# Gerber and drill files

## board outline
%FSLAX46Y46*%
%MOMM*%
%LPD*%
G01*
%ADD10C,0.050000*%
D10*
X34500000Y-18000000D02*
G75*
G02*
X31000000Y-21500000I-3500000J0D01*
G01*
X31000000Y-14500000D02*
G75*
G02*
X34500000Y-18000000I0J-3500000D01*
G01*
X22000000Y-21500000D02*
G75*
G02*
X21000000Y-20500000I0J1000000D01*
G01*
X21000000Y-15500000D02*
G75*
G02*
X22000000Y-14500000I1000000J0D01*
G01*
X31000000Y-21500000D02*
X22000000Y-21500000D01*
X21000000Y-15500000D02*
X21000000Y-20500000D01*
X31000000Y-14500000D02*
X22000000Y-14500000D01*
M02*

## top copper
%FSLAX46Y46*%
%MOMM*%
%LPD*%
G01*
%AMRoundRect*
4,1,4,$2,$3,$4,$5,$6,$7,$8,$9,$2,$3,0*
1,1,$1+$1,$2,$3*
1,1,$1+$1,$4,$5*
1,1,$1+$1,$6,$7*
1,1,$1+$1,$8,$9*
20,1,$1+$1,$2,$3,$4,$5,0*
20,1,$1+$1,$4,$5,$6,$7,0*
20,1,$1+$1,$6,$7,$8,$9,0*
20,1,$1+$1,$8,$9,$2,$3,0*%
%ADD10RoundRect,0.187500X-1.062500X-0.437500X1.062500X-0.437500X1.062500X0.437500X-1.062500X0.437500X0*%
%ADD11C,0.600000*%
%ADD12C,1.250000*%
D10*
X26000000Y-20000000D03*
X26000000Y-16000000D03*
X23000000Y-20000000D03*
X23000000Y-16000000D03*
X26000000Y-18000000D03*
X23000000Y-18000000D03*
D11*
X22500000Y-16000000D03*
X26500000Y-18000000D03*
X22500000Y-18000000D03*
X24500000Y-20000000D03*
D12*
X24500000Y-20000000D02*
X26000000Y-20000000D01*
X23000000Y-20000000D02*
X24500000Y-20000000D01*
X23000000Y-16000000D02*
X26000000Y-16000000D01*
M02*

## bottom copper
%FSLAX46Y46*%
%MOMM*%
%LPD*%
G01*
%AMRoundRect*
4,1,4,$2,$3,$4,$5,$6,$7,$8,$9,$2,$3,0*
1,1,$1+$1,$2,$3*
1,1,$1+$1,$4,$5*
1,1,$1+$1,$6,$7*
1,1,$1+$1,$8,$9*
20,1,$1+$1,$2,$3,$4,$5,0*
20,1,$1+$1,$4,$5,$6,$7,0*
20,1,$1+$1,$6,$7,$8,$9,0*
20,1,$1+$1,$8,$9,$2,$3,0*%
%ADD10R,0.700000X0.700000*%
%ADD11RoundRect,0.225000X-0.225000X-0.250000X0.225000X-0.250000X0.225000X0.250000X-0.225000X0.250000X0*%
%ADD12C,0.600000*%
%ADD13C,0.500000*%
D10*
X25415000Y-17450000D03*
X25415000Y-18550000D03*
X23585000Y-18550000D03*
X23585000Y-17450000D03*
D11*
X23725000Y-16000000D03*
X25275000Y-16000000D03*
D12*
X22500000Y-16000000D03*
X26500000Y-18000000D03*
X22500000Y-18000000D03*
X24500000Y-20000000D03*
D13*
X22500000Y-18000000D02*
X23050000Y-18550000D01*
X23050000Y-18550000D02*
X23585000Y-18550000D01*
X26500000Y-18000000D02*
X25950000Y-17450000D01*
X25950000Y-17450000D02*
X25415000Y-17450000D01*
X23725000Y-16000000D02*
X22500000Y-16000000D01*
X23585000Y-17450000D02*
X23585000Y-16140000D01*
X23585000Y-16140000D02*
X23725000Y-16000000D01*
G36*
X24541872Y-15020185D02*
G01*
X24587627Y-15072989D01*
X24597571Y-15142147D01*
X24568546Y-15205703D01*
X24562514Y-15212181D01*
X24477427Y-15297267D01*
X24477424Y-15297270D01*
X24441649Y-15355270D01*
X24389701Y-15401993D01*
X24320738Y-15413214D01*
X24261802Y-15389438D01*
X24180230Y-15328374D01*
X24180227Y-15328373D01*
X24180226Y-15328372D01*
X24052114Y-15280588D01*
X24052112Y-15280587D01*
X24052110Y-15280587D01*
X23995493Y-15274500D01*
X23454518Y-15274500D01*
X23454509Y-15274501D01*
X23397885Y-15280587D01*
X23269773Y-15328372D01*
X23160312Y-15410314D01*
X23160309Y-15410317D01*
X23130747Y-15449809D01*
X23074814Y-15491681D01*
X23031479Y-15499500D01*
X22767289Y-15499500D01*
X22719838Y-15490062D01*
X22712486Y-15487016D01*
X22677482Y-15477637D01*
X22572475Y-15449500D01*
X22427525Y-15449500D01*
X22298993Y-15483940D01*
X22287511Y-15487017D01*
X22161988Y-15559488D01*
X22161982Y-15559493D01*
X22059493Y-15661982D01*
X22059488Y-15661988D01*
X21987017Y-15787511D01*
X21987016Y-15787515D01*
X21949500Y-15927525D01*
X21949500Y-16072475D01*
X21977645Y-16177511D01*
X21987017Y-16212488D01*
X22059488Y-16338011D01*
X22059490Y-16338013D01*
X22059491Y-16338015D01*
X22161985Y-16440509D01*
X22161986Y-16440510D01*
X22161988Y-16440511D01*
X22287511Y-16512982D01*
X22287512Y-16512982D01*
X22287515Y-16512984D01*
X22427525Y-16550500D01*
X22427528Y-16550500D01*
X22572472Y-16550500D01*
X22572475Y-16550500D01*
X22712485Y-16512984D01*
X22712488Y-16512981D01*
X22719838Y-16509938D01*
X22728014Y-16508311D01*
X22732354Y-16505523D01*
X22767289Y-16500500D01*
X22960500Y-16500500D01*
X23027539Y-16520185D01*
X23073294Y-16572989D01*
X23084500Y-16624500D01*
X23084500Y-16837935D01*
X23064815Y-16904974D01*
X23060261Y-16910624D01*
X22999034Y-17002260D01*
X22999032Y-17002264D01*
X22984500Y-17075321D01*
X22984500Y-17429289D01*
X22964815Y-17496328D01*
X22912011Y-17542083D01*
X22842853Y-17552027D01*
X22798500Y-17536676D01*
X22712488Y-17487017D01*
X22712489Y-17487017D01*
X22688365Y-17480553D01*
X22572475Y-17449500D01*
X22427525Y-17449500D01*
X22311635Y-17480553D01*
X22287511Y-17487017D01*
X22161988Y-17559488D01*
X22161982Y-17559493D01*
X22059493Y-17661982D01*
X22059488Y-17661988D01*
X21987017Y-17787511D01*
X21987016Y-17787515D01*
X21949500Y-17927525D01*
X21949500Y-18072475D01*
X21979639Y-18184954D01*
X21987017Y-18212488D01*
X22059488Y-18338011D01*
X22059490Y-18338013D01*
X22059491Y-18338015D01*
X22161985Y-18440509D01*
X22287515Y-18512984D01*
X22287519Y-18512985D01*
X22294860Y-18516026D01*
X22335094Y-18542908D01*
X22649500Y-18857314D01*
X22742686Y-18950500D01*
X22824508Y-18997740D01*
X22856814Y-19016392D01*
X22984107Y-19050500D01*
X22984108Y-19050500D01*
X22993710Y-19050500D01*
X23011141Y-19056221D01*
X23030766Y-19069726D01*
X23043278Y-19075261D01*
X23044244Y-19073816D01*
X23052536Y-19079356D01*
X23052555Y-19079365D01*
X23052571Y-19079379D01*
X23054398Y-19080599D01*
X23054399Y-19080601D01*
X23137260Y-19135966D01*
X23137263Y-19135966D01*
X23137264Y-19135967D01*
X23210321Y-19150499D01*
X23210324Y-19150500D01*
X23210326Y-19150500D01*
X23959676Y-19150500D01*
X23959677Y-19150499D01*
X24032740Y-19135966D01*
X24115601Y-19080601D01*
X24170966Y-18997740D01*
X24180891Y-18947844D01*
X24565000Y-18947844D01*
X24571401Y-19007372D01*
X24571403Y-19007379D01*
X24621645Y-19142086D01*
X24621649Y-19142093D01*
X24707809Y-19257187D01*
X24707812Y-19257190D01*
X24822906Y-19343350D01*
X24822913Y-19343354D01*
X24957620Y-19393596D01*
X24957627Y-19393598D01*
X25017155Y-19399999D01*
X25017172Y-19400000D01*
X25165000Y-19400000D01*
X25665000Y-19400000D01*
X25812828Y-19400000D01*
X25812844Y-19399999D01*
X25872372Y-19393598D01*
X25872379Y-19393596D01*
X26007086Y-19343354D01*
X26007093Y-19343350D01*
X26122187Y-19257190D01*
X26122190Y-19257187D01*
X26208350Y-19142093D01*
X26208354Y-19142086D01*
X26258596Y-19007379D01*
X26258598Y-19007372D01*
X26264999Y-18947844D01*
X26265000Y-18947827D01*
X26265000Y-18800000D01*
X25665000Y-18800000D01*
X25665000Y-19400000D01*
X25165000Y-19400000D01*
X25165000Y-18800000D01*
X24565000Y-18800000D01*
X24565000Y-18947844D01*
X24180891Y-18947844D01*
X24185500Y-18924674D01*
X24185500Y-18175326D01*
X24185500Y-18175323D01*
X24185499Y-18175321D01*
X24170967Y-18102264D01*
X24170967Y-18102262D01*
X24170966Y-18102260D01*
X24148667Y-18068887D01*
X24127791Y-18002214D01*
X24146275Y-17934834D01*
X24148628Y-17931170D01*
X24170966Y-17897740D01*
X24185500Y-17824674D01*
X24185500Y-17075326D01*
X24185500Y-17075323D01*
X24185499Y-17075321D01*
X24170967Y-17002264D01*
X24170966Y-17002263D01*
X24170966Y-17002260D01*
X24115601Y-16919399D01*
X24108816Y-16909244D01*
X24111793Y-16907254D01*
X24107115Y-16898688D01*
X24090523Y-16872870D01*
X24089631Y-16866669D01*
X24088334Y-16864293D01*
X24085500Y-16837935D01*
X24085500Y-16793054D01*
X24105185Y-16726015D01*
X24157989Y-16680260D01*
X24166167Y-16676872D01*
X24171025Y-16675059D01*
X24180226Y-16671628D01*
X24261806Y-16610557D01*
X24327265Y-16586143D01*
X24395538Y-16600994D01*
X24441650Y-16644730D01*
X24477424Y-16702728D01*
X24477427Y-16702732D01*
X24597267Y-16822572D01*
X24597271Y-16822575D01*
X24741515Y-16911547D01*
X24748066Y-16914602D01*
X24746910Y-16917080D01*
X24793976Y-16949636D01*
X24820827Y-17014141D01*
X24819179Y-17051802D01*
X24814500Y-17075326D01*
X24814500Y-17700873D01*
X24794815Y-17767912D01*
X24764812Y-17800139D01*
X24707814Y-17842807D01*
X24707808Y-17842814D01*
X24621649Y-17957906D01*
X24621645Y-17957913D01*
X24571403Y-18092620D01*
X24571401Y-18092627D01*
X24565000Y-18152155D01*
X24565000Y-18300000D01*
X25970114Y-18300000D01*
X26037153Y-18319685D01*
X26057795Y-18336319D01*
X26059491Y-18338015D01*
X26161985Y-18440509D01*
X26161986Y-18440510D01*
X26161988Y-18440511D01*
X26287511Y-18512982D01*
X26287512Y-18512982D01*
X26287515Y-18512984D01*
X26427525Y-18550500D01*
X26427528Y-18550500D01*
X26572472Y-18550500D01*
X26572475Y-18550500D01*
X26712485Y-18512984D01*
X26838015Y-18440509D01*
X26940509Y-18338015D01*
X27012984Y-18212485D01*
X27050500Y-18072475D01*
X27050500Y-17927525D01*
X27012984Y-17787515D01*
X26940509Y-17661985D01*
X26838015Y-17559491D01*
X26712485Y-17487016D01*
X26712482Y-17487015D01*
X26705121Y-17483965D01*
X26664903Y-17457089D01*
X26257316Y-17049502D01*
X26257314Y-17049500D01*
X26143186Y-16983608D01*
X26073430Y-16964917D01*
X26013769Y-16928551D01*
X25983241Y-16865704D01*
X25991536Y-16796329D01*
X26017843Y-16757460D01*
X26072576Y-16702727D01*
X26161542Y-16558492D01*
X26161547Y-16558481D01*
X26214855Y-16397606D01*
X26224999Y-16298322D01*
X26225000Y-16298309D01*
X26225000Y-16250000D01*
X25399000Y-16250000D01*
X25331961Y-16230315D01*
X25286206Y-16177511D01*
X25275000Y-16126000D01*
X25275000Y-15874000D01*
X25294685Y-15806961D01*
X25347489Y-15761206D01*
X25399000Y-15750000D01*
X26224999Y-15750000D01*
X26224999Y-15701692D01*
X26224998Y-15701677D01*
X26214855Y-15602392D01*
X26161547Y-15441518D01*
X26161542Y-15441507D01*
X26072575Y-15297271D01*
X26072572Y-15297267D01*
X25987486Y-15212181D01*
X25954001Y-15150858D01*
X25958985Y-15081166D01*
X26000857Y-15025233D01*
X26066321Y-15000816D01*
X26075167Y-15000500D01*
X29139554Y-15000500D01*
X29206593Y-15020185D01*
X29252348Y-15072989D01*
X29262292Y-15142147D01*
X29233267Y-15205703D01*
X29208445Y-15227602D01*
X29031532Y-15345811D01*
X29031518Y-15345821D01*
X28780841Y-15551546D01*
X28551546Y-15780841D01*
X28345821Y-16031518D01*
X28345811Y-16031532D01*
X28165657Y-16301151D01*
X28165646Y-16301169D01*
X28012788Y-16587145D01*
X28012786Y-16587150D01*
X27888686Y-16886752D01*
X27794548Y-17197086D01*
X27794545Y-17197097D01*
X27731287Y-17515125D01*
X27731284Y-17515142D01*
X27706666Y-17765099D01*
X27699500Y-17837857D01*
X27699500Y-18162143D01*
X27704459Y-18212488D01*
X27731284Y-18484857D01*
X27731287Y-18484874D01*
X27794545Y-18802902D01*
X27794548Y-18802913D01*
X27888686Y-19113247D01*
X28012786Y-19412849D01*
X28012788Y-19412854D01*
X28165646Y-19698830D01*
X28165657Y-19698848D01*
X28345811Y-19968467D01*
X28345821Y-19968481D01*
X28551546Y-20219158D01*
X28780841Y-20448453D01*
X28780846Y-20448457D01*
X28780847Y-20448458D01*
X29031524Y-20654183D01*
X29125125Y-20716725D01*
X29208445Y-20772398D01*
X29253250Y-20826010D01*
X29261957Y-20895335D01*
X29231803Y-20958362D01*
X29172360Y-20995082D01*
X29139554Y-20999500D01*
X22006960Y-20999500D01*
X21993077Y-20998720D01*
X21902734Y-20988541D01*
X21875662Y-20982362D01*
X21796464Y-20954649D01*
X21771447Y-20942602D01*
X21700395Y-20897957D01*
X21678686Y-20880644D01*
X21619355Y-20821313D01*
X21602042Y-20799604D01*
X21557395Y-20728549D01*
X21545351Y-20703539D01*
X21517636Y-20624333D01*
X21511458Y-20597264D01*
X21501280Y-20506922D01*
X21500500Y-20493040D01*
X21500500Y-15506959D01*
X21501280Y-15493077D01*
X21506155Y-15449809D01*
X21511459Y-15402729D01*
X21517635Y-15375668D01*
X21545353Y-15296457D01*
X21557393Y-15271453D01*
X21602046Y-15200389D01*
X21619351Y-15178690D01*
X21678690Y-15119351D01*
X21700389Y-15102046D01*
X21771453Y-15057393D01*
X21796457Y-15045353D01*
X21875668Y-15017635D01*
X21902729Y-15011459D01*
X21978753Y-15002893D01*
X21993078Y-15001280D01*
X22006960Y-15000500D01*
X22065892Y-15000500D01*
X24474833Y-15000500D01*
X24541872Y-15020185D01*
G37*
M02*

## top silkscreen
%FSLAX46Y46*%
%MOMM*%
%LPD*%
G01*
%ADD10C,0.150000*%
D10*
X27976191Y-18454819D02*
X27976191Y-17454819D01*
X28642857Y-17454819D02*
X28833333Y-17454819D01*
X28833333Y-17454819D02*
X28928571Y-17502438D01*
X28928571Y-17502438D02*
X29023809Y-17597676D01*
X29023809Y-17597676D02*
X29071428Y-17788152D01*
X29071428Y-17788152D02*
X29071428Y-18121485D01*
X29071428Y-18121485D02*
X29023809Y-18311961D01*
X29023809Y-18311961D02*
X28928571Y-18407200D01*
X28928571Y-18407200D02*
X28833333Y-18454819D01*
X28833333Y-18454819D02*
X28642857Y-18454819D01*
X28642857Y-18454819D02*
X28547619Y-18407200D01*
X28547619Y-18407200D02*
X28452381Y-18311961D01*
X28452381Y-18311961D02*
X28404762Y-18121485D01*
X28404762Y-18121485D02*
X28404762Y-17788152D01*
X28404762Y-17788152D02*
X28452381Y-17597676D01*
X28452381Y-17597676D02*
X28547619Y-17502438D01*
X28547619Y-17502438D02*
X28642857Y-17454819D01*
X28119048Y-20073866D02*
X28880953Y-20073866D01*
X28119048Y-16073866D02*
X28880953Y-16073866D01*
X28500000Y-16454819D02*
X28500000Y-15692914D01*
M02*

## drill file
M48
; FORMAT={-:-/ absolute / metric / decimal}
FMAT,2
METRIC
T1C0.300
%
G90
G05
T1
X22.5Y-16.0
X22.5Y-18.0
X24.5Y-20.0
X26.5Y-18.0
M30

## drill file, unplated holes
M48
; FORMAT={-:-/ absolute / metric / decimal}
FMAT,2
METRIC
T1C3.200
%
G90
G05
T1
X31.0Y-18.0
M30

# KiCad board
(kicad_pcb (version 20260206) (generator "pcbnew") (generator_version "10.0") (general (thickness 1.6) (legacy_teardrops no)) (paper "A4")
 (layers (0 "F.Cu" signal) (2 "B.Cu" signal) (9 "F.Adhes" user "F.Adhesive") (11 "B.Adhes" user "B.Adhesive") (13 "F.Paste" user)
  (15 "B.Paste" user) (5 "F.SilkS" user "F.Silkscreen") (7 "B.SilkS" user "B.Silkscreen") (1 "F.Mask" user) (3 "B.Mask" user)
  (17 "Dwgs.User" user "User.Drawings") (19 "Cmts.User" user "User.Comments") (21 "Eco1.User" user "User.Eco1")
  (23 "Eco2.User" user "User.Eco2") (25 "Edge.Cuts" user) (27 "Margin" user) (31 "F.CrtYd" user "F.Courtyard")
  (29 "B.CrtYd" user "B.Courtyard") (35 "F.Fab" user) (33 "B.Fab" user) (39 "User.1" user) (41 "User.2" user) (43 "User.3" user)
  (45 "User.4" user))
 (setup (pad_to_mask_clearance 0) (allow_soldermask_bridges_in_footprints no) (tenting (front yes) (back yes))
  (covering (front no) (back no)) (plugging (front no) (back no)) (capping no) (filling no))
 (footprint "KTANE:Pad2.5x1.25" (layer "F.Cu") (at 26 16)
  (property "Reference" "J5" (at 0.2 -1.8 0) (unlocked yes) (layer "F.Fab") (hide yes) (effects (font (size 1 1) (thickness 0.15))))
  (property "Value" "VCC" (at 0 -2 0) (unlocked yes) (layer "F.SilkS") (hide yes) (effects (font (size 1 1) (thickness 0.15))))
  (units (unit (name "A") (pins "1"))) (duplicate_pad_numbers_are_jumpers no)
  (pad "1" smd roundrect (at 0 0) (size 2.5 1.25) (layers "F.Cu" "F.Mask") (roundrect_rratio 0.15) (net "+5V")))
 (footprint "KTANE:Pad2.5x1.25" (layer "F.Cu") (at 26 18)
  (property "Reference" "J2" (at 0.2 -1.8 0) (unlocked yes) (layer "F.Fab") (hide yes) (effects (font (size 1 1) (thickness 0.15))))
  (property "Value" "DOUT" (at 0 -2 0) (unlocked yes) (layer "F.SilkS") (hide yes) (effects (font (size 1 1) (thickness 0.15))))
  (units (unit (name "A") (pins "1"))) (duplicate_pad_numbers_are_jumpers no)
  (pad "1" smd roundrect (at 0 0) (size 2.5 1.25) (layers "F.Cu" "F.Mask") (roundrect_rratio 0.15) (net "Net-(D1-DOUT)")))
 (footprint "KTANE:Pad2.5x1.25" (layer "F.Cu") (at 23 18)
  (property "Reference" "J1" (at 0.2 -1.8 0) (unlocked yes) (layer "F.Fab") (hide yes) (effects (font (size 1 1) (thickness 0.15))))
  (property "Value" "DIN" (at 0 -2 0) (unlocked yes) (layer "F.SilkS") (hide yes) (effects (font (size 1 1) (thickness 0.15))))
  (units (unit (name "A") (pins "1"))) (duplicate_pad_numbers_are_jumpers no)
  (pad "1" smd roundrect (at 0 0) (size 2.5 1.25) (layers "F.Cu" "F.Mask") (roundrect_rratio 0.15) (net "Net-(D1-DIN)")))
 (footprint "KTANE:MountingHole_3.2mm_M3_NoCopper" (layer "F.Cu") (at 31 18)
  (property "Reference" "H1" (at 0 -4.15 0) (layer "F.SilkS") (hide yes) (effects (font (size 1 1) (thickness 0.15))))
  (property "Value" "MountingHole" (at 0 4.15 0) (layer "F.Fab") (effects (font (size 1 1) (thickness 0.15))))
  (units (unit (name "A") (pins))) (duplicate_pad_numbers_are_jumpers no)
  (pad "" np_thru_hole circle (at 0 0) (size 3.2 3.2) (drill 3.2) (layers "*.Cu" "*.Mask") (clearance 1.7)))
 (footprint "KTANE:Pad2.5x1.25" (layer "F.Cu") (at 23 20)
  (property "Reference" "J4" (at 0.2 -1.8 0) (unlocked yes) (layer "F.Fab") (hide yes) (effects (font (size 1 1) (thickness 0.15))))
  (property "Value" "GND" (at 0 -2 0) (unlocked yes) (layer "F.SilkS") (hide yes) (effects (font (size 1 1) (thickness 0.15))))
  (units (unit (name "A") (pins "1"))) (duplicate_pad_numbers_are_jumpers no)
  (pad "1" smd roundrect (at 0 0) (size 2.5 1.25) (layers "F.Cu" "F.Mask") (roundrect_rratio 0.15) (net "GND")))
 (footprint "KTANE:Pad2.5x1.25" (layer "F.Cu") (at 26 20)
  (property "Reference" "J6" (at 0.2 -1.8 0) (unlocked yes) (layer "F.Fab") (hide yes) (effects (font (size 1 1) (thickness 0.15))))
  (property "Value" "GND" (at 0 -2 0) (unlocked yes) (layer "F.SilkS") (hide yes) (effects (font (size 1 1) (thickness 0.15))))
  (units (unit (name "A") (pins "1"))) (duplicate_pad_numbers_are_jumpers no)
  (pad "1" smd roundrect (at 0 0) (size 2.5 1.25) (layers "F.Cu" "F.Mask") (roundrect_rratio 0.15) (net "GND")))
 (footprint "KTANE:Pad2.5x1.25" (layer "F.Cu") (at 23 16)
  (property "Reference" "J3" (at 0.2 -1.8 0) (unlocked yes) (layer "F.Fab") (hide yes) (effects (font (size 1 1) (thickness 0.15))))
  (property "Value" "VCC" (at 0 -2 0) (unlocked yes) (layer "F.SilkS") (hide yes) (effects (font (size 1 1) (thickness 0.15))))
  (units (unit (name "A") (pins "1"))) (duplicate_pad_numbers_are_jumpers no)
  (pad "1" smd roundrect (at 0 0) (size 2.5 1.25) (layers "F.Cu" "F.Mask") (roundrect_rratio 0.15) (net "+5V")))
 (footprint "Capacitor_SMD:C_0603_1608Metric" (layer "B.Cu") (at 24.5 16)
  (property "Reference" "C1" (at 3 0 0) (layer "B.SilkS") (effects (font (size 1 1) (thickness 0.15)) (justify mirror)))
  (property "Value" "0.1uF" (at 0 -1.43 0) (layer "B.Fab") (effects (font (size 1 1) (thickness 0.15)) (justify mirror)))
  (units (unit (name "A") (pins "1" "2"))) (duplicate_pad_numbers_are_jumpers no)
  (pad "1" smd roundrect (at -0.775 0) (size 0.9 0.95) (layers "B.Cu" "B.Mask" "B.Paste") (roundrect_rratio 0.25) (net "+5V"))
  (pad "2" smd roundrect (at 0.775 0) (size 0.9 0.95) (layers "B.Cu" "B.Mask" "B.Paste") (roundrect_rratio 0.25) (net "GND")))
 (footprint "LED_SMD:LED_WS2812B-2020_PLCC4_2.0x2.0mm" (layer "B.Cu") (at 24.5 18 180)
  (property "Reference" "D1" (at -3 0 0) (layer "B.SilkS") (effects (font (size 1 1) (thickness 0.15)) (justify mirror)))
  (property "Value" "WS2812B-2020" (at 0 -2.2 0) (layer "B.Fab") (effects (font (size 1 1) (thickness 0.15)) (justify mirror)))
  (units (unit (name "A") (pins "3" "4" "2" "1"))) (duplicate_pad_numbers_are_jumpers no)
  (pad "1" smd rect (at -0.915 0.55 180) (size 0.7 0.7) (layers "B.Cu" "B.Mask" "B.Paste") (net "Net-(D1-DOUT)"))
  (pad "2" smd rect (at -0.915 -0.55 180) (size 0.7 0.7) (layers "B.Cu" "B.Mask" "B.Paste") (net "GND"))
  (pad "3" smd rect (at 0.915 -0.55 180) (size 0.7 0.7) (layers "B.Cu" "B.Mask" "B.Paste") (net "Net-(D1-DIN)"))
  (pad "4" smd rect (at 0.915 0.55 180) (size 0.7 0.7) (layers "B.Cu" "B.Mask" "B.Paste") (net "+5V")))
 (gr_line (start 21 15.5) (end 21 20.5) (stroke (width 0.05) (type default)) (layer "Edge.Cuts"))
 (gr_arc (start 21 15.5) (mid 21.292893 14.792893) (end 22 14.5) (stroke (width 0.05) (type default)) (layer "Edge.Cuts"))
 (gr_arc (start 22 21.5) (mid 21.292893 21.207107) (end 21 20.5) (stroke (width 0.05) (type default)) (layer "Edge.Cuts"))
 (gr_line (start 31 14.5) (end 22 14.5) (stroke (width 0.05) (type default)) (layer "Edge.Cuts"))
 (gr_arc (start 31 14.5) (mid 33.474874 15.525126) (end 34.5 18) (stroke (width 0.05) (type default)) (layer "Edge.Cuts"))
 (gr_line (start 31 21.5) (end 22 21.5) (stroke (width 0.05) (type default)) (layer "Edge.Cuts"))
 (gr_arc (start 34.5 18) (mid 33.474874 20.474874) (end 31 21.5) (stroke (width 0.05) (type default)) (layer "Edge.Cuts"))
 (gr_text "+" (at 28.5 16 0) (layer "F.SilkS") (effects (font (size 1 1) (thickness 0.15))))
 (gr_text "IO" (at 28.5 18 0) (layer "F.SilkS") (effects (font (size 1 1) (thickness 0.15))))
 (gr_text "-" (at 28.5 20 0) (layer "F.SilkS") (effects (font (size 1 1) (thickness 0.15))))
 (segment (start 23 16) (end 26 16) (width 1.25) (layer "F.Cu") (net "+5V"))
 (via (at 22.5 16) (size 0.6) (drill 0.3) (layers "F.Cu" "B.Cu") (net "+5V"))
 (segment (start 23.725 16) (end 22.5 16) (width 0.5) (layer "B.Cu") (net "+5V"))
 (segment (start 23.585 17.45) (end 23.585 16.14) (width 0.5) (layer "B.Cu") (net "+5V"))
 (segment (start 23.585 16.14) (end 23.725 16) (width 0.5) (layer "B.Cu") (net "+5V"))
 (segment (start 23 20) (end 24.5 20) (width 1.25) (layer "F.Cu") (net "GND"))
 (segment (start 24.5 20) (end 26 20) (width 1.25) (layer "F.Cu") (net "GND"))
 (via (at 24.5 20) (size 0.6) (drill 0.3) (layers "F.Cu" "B.Cu") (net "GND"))
 (via (at 26.5 18) (size 0.6) (drill 0.3) (layers "F.Cu" "B.Cu") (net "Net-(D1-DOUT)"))
 (segment (start 26.5 18) (end 25.95 17.45) (width 0.5) (layer "B.Cu") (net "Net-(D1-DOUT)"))
 (segment (start 25.95 17.45) (end 25.415 17.45) (width 0.5) (layer "B.Cu") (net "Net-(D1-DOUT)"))
 (via (at 22.5 18) (size 0.6) (drill 0.3) (layers "F.Cu" "B.Cu") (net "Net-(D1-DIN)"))
 (segment (start 23.05 18.55) (end 23.585 18.55) (width 0.5) (layer "B.Cu") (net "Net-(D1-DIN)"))
 (segment (start 22.5 18) (end 23.05 18.55) (width 0.5) (layer "B.Cu") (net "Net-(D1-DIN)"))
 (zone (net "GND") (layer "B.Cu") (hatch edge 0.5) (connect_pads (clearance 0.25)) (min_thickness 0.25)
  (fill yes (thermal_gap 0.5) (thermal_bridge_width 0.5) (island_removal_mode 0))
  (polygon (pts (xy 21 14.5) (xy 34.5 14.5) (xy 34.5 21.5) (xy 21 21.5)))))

